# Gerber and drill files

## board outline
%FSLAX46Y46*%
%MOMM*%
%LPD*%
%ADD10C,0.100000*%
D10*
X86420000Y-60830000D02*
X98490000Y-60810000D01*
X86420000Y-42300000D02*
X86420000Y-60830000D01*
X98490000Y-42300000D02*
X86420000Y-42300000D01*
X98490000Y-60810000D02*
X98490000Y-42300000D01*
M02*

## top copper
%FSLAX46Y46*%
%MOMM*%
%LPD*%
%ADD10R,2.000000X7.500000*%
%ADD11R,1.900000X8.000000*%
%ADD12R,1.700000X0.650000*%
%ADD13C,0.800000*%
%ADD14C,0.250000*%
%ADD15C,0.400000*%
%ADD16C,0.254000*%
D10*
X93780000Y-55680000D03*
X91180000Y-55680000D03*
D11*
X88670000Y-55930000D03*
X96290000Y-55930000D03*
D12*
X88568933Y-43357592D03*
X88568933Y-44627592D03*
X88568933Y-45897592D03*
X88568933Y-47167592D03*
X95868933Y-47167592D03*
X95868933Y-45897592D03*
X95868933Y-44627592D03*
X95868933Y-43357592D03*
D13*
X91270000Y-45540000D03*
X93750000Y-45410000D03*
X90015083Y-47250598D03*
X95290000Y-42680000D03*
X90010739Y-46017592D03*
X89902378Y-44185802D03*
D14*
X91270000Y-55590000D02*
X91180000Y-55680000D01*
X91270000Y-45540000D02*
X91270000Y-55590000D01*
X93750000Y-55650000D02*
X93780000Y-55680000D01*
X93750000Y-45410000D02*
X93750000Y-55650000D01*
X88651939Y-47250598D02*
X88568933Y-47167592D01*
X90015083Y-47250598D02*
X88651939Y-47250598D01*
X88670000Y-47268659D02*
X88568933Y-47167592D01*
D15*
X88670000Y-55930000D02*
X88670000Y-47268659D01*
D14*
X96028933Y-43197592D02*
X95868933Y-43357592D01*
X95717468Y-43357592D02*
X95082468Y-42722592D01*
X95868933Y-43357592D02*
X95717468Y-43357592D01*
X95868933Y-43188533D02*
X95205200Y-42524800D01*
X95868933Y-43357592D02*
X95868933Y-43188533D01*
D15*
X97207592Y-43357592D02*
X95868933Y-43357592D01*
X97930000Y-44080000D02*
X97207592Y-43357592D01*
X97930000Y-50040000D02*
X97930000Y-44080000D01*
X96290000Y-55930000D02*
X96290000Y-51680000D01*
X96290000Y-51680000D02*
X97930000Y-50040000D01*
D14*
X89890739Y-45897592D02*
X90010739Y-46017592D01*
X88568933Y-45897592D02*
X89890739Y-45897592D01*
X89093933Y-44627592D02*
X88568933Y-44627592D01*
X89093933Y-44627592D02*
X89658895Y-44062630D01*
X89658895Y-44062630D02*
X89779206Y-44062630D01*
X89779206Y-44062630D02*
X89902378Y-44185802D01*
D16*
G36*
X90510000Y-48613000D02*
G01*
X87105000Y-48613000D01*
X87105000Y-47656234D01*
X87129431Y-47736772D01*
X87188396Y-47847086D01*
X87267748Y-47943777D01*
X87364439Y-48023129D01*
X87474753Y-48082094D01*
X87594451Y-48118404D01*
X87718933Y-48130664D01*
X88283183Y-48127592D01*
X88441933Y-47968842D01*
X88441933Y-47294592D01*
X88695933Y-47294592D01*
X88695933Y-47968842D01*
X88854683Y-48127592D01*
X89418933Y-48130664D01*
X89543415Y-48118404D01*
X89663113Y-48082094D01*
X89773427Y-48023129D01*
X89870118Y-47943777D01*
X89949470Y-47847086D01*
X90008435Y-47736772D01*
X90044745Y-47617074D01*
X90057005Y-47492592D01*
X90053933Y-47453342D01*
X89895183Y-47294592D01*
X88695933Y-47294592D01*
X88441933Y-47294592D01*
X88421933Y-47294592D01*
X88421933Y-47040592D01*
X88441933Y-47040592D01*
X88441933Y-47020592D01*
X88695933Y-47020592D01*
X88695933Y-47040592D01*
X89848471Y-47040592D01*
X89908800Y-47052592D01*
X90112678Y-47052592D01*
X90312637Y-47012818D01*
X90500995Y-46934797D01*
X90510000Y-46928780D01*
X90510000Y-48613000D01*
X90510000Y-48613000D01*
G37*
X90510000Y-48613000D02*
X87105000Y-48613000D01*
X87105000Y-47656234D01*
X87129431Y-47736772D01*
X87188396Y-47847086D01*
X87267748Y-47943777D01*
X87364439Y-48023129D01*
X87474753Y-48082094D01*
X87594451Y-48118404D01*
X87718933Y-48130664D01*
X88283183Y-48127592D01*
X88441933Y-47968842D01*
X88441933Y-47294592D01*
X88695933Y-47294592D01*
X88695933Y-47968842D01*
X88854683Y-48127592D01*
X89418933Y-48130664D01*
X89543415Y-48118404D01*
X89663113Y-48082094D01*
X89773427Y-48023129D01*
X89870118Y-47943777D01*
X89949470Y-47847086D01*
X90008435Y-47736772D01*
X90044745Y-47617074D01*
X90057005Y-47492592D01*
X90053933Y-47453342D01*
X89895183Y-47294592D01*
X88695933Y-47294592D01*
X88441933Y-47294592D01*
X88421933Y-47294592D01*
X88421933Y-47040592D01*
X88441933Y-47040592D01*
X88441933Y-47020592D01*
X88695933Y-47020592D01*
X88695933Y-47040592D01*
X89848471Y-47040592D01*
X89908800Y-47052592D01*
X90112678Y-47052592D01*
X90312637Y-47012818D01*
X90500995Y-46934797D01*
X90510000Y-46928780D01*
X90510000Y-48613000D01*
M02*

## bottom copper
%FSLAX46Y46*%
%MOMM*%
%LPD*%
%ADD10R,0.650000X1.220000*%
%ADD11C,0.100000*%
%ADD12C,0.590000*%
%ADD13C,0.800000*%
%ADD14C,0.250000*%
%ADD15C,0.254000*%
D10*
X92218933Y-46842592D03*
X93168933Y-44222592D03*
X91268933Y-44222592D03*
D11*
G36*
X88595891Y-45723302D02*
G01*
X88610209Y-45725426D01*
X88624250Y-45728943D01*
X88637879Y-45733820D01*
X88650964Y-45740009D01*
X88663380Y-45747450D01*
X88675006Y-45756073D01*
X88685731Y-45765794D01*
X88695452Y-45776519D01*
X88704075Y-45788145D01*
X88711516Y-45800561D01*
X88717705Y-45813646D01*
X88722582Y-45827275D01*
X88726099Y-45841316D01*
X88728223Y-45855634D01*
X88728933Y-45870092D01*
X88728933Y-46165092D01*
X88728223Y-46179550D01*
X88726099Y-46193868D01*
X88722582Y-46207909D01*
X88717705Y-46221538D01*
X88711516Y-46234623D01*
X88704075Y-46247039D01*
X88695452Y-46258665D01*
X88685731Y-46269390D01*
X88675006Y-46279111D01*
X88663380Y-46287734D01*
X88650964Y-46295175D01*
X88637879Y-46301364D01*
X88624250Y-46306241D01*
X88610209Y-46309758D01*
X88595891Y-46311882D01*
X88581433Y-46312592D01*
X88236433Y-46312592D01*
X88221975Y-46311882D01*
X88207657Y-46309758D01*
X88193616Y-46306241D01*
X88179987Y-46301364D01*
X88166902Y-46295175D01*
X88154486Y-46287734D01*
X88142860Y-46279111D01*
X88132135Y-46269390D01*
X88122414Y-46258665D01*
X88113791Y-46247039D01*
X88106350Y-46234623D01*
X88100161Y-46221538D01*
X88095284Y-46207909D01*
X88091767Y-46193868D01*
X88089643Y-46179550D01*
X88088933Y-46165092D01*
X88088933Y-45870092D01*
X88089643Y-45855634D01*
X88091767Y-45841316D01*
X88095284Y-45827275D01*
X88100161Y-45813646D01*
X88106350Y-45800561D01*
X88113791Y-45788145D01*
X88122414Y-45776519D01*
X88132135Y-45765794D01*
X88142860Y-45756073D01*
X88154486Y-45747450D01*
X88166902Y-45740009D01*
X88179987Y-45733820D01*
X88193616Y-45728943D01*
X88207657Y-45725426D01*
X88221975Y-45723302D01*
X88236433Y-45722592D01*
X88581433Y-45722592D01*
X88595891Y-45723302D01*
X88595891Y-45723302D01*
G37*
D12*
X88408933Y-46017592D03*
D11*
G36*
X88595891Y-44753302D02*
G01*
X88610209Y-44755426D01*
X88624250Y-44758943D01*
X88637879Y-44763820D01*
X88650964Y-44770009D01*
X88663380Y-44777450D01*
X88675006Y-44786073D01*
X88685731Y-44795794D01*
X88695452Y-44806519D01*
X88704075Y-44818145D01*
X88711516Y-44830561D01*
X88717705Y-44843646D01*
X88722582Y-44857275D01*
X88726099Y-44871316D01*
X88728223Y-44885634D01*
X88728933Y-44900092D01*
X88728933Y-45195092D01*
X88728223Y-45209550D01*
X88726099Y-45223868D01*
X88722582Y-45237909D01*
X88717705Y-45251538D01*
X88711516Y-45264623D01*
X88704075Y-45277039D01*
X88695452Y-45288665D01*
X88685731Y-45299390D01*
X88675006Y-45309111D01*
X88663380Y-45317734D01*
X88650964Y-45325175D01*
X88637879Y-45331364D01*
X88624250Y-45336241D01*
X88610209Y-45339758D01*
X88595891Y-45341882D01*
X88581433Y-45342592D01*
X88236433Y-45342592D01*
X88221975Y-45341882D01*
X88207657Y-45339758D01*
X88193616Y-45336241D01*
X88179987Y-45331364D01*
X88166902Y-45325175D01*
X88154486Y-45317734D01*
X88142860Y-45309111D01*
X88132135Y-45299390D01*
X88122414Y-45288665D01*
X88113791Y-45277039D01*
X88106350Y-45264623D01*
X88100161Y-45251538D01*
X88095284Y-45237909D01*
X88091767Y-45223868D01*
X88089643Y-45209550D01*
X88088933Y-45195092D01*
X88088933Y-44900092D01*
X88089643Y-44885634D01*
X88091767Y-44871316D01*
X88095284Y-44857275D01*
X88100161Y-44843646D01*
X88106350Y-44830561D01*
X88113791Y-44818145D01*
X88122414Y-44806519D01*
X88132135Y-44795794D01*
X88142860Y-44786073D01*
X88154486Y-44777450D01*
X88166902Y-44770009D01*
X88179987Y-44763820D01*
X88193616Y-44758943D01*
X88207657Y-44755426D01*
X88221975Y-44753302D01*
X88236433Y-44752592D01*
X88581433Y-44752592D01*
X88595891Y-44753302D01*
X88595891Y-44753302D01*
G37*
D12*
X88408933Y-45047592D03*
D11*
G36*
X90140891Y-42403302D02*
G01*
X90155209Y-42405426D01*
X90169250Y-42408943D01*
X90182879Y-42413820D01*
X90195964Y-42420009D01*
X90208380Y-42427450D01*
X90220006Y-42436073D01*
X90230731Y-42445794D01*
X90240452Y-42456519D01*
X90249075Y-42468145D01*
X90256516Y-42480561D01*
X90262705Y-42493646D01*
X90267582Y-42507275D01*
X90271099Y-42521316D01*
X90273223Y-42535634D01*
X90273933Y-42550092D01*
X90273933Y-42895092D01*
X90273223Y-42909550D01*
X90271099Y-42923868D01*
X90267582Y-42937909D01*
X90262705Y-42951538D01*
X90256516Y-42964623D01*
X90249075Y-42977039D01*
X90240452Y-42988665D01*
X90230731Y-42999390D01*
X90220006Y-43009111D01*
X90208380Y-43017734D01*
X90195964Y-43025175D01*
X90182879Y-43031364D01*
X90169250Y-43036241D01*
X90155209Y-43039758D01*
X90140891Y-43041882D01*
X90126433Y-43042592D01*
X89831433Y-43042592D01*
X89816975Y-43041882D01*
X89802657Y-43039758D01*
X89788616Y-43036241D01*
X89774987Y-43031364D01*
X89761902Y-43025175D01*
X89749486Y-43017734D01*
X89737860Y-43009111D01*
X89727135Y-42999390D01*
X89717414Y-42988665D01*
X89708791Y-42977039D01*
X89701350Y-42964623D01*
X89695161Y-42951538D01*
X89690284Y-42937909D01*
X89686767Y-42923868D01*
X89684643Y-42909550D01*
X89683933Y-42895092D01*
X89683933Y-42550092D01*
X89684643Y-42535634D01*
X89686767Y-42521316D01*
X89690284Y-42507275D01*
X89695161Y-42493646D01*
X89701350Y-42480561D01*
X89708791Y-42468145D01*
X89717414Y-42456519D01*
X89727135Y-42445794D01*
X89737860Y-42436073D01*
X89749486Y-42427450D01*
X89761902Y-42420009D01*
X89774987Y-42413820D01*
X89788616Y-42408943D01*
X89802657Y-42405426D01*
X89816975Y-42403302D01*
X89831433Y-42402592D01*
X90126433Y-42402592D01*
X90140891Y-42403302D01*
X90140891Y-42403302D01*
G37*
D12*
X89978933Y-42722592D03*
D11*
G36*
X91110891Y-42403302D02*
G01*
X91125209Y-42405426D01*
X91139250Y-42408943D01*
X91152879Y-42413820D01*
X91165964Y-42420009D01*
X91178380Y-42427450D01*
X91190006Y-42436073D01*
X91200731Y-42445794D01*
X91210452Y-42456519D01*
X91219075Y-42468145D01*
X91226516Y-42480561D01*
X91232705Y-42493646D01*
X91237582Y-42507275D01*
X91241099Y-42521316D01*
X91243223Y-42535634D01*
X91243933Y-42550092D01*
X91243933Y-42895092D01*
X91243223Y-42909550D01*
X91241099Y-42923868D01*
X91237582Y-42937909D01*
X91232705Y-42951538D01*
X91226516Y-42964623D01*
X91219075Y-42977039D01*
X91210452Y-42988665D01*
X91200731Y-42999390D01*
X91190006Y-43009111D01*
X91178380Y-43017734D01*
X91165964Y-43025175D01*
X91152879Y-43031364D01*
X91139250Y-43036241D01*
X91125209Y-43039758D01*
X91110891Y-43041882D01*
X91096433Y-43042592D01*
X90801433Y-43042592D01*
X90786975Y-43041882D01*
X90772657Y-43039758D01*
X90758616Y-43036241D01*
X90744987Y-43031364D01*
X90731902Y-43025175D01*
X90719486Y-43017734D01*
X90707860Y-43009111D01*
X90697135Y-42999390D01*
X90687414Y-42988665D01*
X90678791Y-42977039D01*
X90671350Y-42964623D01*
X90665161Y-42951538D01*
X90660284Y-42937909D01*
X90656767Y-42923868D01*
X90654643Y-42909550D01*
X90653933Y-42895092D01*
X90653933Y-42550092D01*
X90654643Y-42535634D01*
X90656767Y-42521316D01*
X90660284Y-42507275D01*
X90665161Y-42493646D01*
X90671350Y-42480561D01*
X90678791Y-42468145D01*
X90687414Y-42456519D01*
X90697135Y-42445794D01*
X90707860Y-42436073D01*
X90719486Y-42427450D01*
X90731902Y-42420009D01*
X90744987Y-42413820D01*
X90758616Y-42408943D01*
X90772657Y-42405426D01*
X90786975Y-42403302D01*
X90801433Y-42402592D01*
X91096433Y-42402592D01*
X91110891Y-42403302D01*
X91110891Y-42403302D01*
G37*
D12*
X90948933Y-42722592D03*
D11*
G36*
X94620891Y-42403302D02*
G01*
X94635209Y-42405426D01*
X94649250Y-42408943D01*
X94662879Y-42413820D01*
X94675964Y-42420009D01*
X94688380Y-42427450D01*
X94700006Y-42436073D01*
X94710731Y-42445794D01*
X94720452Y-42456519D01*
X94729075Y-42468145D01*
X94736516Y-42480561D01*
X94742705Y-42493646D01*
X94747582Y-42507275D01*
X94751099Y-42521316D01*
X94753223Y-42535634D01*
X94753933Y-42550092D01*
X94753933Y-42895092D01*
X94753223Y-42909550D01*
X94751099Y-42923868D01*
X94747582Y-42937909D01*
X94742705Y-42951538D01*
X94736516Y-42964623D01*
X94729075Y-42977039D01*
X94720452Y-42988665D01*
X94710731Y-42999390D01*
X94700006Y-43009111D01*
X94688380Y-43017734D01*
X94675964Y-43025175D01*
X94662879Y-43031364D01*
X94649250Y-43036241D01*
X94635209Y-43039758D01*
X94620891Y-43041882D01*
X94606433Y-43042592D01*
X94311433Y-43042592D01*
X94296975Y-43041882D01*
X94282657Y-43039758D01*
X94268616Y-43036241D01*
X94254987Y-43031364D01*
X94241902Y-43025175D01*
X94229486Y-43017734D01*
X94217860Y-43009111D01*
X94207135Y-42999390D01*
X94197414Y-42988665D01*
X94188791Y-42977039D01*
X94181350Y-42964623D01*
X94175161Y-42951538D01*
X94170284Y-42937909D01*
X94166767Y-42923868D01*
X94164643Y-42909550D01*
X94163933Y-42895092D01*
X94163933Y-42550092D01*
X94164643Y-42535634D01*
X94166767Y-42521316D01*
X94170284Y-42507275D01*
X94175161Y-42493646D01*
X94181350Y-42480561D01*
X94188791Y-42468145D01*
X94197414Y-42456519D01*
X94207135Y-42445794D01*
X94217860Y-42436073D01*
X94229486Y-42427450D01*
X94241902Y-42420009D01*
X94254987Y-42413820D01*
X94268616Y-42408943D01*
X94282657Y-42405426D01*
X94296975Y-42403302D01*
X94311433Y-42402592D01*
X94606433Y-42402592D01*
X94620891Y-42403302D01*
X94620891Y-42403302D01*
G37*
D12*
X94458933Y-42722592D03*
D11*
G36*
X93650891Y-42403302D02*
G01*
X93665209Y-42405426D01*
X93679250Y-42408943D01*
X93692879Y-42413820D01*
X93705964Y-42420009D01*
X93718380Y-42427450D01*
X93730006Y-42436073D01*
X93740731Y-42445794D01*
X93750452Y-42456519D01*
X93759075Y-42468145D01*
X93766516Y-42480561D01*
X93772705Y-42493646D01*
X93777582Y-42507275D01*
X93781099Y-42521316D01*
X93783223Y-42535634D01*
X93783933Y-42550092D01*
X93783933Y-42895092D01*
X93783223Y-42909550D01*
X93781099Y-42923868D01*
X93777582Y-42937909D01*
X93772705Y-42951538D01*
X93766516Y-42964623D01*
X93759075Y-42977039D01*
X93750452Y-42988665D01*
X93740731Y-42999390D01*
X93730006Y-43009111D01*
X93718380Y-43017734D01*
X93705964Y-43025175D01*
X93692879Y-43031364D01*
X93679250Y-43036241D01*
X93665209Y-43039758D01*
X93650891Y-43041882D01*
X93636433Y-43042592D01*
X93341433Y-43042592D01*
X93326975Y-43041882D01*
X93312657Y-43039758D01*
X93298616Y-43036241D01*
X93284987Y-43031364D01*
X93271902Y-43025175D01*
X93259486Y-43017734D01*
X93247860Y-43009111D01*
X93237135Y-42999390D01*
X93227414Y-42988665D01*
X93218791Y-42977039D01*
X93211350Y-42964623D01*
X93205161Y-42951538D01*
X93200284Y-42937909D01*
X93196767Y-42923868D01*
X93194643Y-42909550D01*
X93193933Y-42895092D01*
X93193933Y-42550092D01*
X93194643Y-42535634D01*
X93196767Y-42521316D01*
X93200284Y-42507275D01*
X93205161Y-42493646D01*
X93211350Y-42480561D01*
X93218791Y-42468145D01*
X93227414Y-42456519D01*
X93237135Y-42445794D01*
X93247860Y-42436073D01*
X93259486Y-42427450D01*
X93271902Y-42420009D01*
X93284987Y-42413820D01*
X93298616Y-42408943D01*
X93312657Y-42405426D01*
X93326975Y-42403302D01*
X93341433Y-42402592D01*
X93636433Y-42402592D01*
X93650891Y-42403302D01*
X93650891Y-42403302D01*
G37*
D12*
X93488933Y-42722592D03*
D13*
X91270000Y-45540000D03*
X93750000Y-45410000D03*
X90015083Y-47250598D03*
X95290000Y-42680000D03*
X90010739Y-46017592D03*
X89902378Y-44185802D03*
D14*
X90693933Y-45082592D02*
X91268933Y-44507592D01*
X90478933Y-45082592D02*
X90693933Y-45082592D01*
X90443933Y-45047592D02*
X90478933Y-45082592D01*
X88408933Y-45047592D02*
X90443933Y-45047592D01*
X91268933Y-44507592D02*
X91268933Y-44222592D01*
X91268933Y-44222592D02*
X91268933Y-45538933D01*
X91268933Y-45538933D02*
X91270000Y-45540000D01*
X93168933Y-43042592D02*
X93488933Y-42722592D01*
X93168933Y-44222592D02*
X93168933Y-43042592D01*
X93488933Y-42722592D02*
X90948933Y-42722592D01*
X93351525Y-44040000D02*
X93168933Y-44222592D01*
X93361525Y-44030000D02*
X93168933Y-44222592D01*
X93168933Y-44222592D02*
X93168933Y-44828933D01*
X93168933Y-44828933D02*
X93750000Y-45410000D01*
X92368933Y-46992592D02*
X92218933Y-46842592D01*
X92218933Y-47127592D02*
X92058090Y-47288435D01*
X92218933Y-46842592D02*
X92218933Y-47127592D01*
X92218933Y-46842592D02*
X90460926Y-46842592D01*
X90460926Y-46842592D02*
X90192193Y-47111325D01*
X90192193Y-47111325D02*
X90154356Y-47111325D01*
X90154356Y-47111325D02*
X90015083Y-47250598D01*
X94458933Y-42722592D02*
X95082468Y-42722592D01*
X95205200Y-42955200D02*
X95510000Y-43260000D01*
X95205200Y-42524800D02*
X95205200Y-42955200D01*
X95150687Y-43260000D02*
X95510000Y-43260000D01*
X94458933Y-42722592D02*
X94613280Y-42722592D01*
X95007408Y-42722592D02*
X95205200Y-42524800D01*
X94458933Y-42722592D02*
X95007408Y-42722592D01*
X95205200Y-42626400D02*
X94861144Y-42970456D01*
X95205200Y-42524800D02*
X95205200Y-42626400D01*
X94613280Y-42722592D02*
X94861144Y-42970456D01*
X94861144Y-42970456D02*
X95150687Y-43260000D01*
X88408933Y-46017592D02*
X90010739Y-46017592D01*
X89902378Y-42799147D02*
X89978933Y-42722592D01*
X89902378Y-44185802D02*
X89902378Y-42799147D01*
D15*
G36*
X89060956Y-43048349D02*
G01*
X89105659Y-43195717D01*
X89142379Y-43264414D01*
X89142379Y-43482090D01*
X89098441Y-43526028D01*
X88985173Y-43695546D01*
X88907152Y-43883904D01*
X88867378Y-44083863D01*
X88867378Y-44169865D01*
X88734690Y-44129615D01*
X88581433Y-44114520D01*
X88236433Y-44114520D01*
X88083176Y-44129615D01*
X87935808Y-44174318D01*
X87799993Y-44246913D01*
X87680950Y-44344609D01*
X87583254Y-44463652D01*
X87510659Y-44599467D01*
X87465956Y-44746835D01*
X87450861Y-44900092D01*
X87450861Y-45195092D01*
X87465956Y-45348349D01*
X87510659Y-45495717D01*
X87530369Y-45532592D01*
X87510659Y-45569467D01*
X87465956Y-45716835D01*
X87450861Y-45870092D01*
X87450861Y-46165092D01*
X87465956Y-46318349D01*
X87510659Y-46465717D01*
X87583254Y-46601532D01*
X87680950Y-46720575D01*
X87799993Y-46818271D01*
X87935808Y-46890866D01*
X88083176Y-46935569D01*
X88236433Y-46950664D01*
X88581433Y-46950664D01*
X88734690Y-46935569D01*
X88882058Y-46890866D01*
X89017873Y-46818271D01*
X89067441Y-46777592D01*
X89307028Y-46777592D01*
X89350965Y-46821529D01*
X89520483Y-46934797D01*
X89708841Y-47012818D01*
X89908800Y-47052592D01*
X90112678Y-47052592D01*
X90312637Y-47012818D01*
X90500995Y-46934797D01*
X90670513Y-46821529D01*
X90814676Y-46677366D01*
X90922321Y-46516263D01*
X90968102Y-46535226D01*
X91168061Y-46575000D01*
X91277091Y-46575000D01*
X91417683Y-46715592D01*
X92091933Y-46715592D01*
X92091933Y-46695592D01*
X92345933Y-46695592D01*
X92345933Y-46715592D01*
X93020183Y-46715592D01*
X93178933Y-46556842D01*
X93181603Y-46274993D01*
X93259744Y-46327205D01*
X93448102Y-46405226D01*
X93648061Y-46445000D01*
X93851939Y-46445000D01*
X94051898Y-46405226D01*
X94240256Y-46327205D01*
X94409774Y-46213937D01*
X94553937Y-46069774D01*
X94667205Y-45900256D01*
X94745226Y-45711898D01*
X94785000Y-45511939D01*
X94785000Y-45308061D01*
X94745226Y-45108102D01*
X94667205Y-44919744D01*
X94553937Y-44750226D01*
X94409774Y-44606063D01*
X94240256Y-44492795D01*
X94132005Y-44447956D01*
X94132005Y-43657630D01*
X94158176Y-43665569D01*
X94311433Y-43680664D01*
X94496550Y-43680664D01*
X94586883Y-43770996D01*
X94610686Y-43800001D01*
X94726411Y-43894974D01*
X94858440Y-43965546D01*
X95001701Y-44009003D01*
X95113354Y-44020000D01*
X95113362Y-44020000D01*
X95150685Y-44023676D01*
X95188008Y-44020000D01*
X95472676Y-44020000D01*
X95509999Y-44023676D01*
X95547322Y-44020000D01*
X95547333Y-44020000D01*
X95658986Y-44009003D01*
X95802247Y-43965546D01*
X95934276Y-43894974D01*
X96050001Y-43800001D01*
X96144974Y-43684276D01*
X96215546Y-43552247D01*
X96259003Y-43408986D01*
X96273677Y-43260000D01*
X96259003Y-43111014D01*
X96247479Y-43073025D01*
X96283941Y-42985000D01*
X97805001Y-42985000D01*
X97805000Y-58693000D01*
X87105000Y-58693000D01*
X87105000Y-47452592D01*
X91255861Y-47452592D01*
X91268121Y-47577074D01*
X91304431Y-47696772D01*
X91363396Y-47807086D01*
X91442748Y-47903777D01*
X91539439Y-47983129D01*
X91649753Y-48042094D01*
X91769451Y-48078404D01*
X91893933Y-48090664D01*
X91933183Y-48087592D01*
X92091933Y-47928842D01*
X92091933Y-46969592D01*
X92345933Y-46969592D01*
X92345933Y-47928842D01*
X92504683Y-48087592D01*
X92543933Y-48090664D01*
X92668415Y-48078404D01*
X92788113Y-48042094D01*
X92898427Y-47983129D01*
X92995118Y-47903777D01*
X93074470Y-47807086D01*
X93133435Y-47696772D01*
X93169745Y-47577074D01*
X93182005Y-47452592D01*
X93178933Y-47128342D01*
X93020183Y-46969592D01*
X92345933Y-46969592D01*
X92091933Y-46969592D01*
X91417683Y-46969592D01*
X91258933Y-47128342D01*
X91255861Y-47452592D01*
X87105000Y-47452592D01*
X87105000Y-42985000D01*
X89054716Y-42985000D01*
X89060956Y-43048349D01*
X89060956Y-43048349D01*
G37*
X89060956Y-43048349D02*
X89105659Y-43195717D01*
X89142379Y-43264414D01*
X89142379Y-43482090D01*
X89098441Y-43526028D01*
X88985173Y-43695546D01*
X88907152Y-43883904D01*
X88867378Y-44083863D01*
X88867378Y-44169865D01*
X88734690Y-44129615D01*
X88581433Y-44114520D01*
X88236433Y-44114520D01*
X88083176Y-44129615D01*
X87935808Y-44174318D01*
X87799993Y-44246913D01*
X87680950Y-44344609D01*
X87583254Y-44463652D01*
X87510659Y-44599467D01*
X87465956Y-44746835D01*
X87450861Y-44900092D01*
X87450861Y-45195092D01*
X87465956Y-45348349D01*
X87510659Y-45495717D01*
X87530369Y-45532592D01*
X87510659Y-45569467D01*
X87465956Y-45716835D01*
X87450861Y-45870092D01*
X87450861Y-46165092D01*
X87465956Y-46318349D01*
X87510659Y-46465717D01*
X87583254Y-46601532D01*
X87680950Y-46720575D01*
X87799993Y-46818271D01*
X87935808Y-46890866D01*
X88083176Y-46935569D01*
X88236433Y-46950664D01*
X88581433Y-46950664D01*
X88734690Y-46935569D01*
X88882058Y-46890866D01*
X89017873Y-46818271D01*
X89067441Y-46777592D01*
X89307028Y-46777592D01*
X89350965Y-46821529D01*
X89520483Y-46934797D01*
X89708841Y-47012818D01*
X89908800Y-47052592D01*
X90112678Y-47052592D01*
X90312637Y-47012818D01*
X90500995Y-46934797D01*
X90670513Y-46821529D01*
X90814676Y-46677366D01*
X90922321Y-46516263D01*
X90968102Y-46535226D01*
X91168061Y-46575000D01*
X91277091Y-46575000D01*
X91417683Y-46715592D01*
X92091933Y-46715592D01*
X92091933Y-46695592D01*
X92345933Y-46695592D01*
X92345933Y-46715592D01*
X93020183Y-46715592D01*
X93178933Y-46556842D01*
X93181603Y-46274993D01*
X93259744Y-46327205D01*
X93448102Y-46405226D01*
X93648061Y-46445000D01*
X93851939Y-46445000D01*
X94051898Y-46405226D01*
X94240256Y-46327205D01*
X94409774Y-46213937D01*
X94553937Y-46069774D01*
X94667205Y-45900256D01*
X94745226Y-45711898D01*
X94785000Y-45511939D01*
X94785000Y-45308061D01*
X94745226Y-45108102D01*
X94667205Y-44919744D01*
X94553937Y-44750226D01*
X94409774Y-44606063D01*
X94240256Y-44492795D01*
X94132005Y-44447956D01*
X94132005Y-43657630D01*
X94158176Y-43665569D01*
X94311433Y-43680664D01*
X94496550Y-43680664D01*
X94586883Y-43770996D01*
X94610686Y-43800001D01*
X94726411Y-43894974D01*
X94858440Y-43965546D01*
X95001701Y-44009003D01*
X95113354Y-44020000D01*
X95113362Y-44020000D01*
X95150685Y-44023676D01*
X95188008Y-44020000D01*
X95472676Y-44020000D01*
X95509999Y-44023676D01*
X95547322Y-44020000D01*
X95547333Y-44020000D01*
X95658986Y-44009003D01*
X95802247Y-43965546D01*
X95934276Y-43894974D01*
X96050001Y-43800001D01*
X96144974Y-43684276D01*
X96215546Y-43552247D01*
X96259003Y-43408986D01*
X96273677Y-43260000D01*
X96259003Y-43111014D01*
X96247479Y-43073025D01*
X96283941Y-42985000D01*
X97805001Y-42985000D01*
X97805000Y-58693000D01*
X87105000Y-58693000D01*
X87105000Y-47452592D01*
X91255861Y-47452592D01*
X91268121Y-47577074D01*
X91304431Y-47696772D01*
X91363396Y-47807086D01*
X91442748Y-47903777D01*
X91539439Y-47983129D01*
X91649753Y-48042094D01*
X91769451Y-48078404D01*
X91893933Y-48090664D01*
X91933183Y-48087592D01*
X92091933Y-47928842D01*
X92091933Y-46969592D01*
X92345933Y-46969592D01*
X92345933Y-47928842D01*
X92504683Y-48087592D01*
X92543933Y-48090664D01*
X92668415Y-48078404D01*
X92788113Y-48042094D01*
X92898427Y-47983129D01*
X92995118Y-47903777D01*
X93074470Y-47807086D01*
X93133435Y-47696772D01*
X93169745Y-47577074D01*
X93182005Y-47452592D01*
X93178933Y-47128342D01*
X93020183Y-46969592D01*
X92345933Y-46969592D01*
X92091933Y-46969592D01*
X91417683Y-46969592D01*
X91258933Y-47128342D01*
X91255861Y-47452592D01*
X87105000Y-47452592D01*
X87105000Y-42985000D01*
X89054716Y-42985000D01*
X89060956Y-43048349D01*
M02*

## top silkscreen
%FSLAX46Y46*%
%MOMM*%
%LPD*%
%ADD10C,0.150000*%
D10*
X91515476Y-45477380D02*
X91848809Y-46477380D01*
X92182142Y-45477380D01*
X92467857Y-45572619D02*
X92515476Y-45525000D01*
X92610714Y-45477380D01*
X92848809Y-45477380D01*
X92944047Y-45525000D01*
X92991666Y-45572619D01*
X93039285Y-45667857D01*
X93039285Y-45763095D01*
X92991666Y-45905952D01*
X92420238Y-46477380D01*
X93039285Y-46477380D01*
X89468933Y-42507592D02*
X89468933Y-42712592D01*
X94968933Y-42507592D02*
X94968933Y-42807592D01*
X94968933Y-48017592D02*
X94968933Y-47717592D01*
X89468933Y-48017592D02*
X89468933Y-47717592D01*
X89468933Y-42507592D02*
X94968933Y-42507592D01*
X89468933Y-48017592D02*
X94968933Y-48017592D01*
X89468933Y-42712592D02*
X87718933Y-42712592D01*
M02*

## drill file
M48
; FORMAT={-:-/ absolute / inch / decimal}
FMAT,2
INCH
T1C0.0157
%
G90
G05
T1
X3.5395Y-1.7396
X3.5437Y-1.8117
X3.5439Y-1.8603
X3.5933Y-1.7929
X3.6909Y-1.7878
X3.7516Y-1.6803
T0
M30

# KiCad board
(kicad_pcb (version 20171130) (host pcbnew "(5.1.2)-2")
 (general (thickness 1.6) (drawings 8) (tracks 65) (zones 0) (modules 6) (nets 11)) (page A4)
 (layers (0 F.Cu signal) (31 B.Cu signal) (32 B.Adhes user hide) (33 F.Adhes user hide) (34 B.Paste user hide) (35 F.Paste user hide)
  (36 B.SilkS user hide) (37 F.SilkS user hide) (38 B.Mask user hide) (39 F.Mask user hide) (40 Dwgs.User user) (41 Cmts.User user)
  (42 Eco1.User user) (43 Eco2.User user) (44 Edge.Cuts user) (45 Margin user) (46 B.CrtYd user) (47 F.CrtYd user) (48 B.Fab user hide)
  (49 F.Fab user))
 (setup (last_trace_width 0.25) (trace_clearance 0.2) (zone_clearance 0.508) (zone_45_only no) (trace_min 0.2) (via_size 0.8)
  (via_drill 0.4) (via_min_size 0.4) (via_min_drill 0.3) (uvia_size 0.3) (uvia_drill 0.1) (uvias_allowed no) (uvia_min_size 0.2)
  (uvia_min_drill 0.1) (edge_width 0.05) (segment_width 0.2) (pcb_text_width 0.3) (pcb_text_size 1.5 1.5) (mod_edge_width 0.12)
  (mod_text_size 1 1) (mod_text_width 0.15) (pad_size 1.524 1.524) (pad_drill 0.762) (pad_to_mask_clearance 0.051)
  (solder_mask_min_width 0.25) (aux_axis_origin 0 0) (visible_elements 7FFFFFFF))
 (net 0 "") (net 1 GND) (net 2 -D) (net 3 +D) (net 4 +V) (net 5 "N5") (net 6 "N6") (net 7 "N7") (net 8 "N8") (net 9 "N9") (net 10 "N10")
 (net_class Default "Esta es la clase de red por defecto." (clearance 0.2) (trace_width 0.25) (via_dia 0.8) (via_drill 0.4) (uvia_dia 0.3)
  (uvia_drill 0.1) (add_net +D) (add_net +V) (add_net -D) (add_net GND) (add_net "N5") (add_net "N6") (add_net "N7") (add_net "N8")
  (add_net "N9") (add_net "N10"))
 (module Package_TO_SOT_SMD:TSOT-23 (layer B.Cu) (at 92.218933 45.532592 270)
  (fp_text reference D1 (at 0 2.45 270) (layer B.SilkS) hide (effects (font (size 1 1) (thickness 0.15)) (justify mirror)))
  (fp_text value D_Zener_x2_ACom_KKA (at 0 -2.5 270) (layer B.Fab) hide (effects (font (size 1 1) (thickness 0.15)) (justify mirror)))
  (pad 3 smd rect (at 1.31 0 270) (size 1.22 0.65) (layers B.Cu B.Paste B.Mask) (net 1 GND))
  (pad 2 smd rect (at -1.31 -0.95 270) (size 1.22 0.65) (layers B.Cu B.Paste B.Mask) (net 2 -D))
  (pad 1 smd rect (at -1.31 0.95 270) (size 1.22 0.65) (layers B.Cu B.Paste B.Mask) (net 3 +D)))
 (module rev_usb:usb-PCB (layer F.Cu) (at 92.48 60.83)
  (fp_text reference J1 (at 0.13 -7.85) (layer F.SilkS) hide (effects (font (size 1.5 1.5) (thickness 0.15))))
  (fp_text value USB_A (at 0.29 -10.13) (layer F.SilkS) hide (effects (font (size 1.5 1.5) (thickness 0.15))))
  (pad 2 connect rect (at 1.3 -5.15) (size 2 7.5) (layers F.Cu F.Mask) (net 2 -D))
  (pad 3 connect rect (at -1.3 -5.15) (size 2 7.5) (layers F.Cu F.Mask) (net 3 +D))
  (pad 4 connect rect (at -3.81 -4.9) (size 1.9 8) (layers F.Cu F.Mask) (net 1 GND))
  (pad 1 connect rect (at 3.81 -4.9) (size 1.9 8) (layers F.Cu F.Mask) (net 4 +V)))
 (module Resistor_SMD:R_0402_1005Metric (layer B.Cu) (at 88.408933 45.532592 90)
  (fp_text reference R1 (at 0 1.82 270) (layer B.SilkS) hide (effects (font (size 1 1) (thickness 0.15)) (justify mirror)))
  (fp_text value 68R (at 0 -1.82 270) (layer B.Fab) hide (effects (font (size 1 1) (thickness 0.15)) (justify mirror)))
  (pad 1 smd roundrect (at -0.485 0 90) (size 0.59 0.64) (layers B.Cu B.Paste B.Mask) (roundrect_rratio 0.25) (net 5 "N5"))
  (pad 2 smd roundrect (at 0.485 0 90) (size 0.59 0.64) (layers B.Cu B.Paste B.Mask) (roundrect_rratio 0.25) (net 3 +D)))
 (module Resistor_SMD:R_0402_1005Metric (layer B.Cu) (at 90.463933 42.722592)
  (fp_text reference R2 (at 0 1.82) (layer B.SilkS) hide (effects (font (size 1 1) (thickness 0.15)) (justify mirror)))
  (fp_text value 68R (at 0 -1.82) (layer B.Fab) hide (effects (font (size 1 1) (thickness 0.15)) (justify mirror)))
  (pad 1 smd roundrect (at -0.485 0) (size 0.59 0.64) (layers B.Cu B.Paste B.Mask) (roundrect_rratio 0.25) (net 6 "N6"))
  (pad 2 smd roundrect (at 0.485 0) (size 0.59 0.64) (layers B.Cu B.Paste B.Mask) (roundrect_rratio 0.25) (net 2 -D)))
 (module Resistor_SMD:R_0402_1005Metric (layer B.Cu) (at 93.973933 42.722592 180)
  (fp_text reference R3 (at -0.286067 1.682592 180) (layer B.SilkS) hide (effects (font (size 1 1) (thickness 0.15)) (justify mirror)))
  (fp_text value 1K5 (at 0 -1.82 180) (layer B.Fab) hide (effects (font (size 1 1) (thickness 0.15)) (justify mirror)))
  (pad 1 smd roundrect (at -0.485 0 180) (size 0.59 0.64) (layers B.Cu B.Paste B.Mask) (roundrect_rratio 0.25) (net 4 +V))
  (pad 2 smd roundrect (at 0.485 0 180) (size 0.59 0.64) (layers B.Cu B.Paste B.Mask) (roundrect_rratio 0.25) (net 2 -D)))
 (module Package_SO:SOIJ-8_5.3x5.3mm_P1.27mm (layer F.Cu) (at 92.218933 45.262592)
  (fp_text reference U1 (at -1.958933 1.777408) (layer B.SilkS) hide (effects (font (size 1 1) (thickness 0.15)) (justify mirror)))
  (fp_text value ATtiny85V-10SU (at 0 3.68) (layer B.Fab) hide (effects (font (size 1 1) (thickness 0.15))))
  (fp_line (start -2.75 -2.755) (end -2.75 -2.55) (layer F.SilkS) (width 0.15))
  (fp_line (start 2.75 -2.755) (end 2.75 -2.455) (layer F.SilkS) (width 0.15))
  (fp_line (start 2.75 2.755) (end 2.75 2.455) (layer F.SilkS) (width 0.15))
  (fp_line (start -2.75 2.755) (end -2.75 2.455) (layer F.SilkS) (width 0.15))
  (fp_line (start -2.75 -2.755) (end 2.75 -2.755) (layer F.SilkS) (width 0.15))
  (fp_line (start -2.75 2.755) (end 2.75 2.755) (layer F.SilkS) (width 0.15))
  (fp_line (start -2.75 -2.55) (end -4.5 -2.55) (layer F.SilkS) (width 0.15))
  (pad 1 smd rect (at -3.65 -1.905) (size 1.7 0.65) (layers F.Cu F.Paste F.Mask) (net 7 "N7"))
  (pad 2 smd rect (at -3.65 -0.635) (size 1.7 0.65) (layers F.Cu F.Paste F.Mask) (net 6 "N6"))
  (pad 3 smd rect (at -3.65 0.635) (size 1.7 0.65) (layers F.Cu F.Paste F.Mask) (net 5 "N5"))
  (pad 4 smd rect (at -3.65 1.905) (size 1.7 0.65) (layers F.Cu F.Paste F.Mask) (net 1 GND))
  (pad 5 smd rect (at 3.65 1.905) (size 1.7 0.65) (layers F.Cu F.Paste F.Mask) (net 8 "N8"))
  (pad 6 smd rect (at 3.65 0.635) (size 1.7 0.65) (layers F.Cu F.Paste F.Mask) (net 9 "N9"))
  (pad 7 smd rect (at 3.65 -0.635) (size 1.7 0.65) (layers F.Cu F.Paste F.Mask) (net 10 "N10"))
  (pad 8 smd rect (at 3.65 -1.905) (size 1.7 0.65) (layers F.Cu F.Paste F.Mask) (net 4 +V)))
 (gr_line (start 86.42 60.83) (end 98.49 60.81) (layer Edge.Cuts) (width 0.1))
 (gr_line (start 86.42 42.3) (end 86.42 60.83) (layer Edge.Cuts) (width 0.1))
 (gr_line (start 98.49 42.3) (end 86.42 42.3) (layer Edge.Cuts) (width 0.1))
 (gr_line (start 98.49 60.81) (end 98.49 42.3) (layer Edge.Cuts) (width 0.1))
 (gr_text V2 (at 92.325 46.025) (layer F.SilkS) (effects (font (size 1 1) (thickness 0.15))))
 (segment (start 90.693933 45.082592) (end 91.268933 44.507592) (width 0.25) (layer B.Cu) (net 3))
 (segment (start 90.478933 45.082592) (end 90.693933 45.082592) (width 0.25) (layer B.Cu) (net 3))
 (segment (start 90.443933 45.047592) (end 90.478933 45.082592) (width 0.25) (layer B.Cu) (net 3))
 (segment (start 88.408933 45.047592) (end 90.443933 45.047592) (width 0.25) (layer B.Cu) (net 3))
 (segment (start 91.268933 44.507592) (end 91.268933 44.222592) (width 0.25) (layer B.Cu) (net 3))
 (via (at 91.27 45.54) (size 0.8) (drill 0.4) (layers F.Cu B.Cu) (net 3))
 (segment (start 91.268933 44.222592) (end 91.268933 45.538933) (width 0.25) (layer B.Cu) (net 3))
 (segment (start 91.268933 45.538933) (end 91.27 45.54) (width 0.25) (layer B.Cu) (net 3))
 (segment (start 91.27 55.59) (end 91.18 55.68) (width 0.25) (layer F.Cu) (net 3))
 (segment (start 91.27 45.54) (end 91.27 55.59) (width 0.25) (layer F.Cu) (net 3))
 (segment (start 93.168933 43.042592) (end 93.488933 42.722592) (width 0.25) (layer B.Cu) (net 2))
 (segment (start 93.168933 44.222592) (end 93.168933 43.042592) (width 0.25) (layer B.Cu) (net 2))
 (segment (start 93.488933 42.722592) (end 90.948933 42.722592) (width 0.25) (layer B.Cu) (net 2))
 (segment (start 93.351525 44.04) (end 93.168933 44.222592) (width 0.25) (layer B.Cu) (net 2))
 (segment (start 93.361525 44.03) (end 93.168933 44.222592) (width 0.25) (layer B.Cu) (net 2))
 (via (at 93.75 45.41) (size 0.8) (drill 0.4) (layers F.Cu B.Cu) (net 2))
 (segment (start 93.168933 44.222592) (end 93.168933 44.828933) (width 0.25) (layer B.Cu) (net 2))
 (segment (start 93.168933 44.828933) (end 93.75 45.41) (width 0.25) (layer B.Cu) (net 2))
 (segment (start 93.75 55.65) (end 93.78 55.68) (width 0.25) (layer F.Cu) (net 2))
 (segment (start 93.75 45.41) (end 93.75 55.65) (width 0.25) (layer F.Cu) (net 2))
 (segment (start 92.368933 46.992592) (end 92.218933 46.842592) (width 0.25) (layer B.Cu) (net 1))
 (segment (start 92.218933 47.127592) (end 92.05809 47.288435) (width 0.25) (layer B.Cu) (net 1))
 (segment (start 92.218933 46.842592) (end 92.218933 47.127592) (width 0.25) (layer B.Cu) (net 1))
 (segment (start 92.218933 46.842592) (end 90.460926 46.842592) (width 0.25) (layer B.Cu) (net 1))
 (segment (start 90.460926 46.842592) (end 90.192193 47.111325) (width 0.25) (layer B.Cu) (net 1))
 (via (at 90.015083 47.250598) (size 0.8) (drill 0.4) (layers F.Cu B.Cu) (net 1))
 (segment (start 90.192193 47.111325) (end 90.154356 47.111325) (width 0.25) (layer B.Cu) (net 1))
 (segment (start 90.154356 47.111325) (end 90.015083 47.250598) (width 0.25) (layer B.Cu) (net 1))
 (segment (start 88.651939 47.250598) (end 88.568933 47.167592) (width 0.25) (layer F.Cu) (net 1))
 (segment (start 90.015083 47.250598) (end 88.651939 47.250598) (width 0.25) (layer F.Cu) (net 1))
 (segment (start 88.67 47.268659) (end 88.568933 47.167592) (width 0.25) (layer F.Cu) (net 1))
 (segment (start 88.67 55.93) (end 88.67 47.268659) (width 0.4) (layer F.Cu) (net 1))
 (segment (start 96.028933 43.197592) (end 95.868933 43.357592) (width 0.25) (layer F.Cu) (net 4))
 (segment (start 94.458933 42.722592) (end 95.082468 42.722592) (width 0.25) (layer B.Cu) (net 4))
 (via (at 95.29 42.68) (size 0.8) (drill 0.4) (layers F.Cu B.Cu) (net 4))
 (segment (start 95.717468 43.357592) (end 95.082468 42.722592) (width 0.25) (layer F.Cu) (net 4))
 (segment (start 95.868933 43.357592) (end 95.717468 43.357592) (width 0.25) (layer F.Cu) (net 4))
 (segment (start 95.868933 43.188533) (end 95.2052 42.5248) (width 0.25) (layer F.Cu) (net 4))
 (segment (start 95.868933 43.357592) (end 95.868933 43.188533) (width 0.25) (layer F.Cu) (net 4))
 (segment (start 95.2052 42.9552) (end 95.51 43.26) (width 0.25) (layer B.Cu) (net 4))
 (segment (start 95.2052 42.5248) (end 95.2052 42.9552) (width 0.25) (layer B.Cu) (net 4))
 (segment (start 95.150687 43.26) (end 95.51 43.26) (width 0.25) (layer B.Cu) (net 4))
 (segment (start 94.458933 42.722592) (end 94.61328 42.722592) (width 0.25) (layer B.Cu) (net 4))
 (segment (start 95.007408 42.722592) (end 95.2052 42.5248) (width 0.25) (layer B.Cu) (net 4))
 (segment (start 94.458933 42.722592) (end 95.007408 42.722592) (width 0.25) (layer B.Cu) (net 4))
 (segment (start 95.2052 42.6264) (end 94.861144 42.970456) (width 0.25) (layer B.Cu) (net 4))
 (segment (start 95.2052 42.5248) (end 95.2052 42.6264) (width 0.25) (layer B.Cu) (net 4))
 (segment (start 94.61328 42.722592) (end 94.861144 42.970456) (width 0.25) (layer B.Cu) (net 4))
 (segment (start 94.861144 42.970456) (end 95.150687 43.26) (width 0.25) (layer B.Cu) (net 4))
 (segment (start 97.207592 43.357592) (end 95.868933 43.357592) (width 0.4) (layer F.Cu) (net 4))
 (segment (start 97.93 44.08) (end 97.207592 43.357592) (width 0.4) (layer F.Cu) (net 4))
 (segment (start 97.93 50.04) (end 97.93 44.08) (width 0.4) (layer F.Cu) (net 4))
 (segment (start 96.29 55.93) (end 96.29 51.68) (width 0.4) (layer F.Cu) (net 4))
 (segment (start 96.29 51.68) (end 97.93 50.04) (width 0.4) (layer F.Cu) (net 4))
 (segment (start 88.408933 46.017592) (end 90.010739 46.017592) (width 0.25) (layer B.Cu) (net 5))
 (via (at 90.010739 46.017592) (size 0.8) (drill 0.4) (layers F.Cu B.Cu) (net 5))
 (segment (start 89.890739 45.897592) (end 90.010739 46.017592) (width 0.25) (layer F.Cu) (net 5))
 (segment (start 88.568933 45.897592) (end 89.890739 45.897592) (width 0.25) (layer F.Cu) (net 5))
 (segment (start 89.093933 44.627592) (end 88.568933 44.627592) (width 0.25) (layer F.Cu) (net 6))
 (segment (start 89.093933 44.627592) (end 89.658895 44.06263) (width 0.25) (layer F.Cu) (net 6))
 (via (at 89.902378 44.185802) (size 0.8) (drill 0.4) (layers F.Cu B.Cu) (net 6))
 (segment (start 89.658895 44.06263) (end 89.779206 44.06263) (width 0.25) (layer F.Cu) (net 6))
 (segment (start 89.779206 44.06263) (end 89.902378 44.185802) (width 0.25) (layer F.Cu) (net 6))
 (segment (start 89.902378 42.799147) (end 89.978933 42.722592) (width 0.25) (layer B.Cu) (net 6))
 (segment (start 89.902378 44.185802) (end 89.902378 42.799147) (width 0.25) (layer B.Cu) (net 6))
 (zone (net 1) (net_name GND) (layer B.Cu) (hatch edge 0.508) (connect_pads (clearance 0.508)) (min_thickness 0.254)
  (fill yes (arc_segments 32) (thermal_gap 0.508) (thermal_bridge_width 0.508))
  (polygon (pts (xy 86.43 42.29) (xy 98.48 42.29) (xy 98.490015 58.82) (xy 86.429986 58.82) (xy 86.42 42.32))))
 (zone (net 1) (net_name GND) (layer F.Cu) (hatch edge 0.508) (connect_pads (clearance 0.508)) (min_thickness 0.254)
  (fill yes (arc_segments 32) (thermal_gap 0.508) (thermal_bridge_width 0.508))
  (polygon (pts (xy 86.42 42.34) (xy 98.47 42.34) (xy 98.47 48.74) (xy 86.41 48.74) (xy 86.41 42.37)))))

